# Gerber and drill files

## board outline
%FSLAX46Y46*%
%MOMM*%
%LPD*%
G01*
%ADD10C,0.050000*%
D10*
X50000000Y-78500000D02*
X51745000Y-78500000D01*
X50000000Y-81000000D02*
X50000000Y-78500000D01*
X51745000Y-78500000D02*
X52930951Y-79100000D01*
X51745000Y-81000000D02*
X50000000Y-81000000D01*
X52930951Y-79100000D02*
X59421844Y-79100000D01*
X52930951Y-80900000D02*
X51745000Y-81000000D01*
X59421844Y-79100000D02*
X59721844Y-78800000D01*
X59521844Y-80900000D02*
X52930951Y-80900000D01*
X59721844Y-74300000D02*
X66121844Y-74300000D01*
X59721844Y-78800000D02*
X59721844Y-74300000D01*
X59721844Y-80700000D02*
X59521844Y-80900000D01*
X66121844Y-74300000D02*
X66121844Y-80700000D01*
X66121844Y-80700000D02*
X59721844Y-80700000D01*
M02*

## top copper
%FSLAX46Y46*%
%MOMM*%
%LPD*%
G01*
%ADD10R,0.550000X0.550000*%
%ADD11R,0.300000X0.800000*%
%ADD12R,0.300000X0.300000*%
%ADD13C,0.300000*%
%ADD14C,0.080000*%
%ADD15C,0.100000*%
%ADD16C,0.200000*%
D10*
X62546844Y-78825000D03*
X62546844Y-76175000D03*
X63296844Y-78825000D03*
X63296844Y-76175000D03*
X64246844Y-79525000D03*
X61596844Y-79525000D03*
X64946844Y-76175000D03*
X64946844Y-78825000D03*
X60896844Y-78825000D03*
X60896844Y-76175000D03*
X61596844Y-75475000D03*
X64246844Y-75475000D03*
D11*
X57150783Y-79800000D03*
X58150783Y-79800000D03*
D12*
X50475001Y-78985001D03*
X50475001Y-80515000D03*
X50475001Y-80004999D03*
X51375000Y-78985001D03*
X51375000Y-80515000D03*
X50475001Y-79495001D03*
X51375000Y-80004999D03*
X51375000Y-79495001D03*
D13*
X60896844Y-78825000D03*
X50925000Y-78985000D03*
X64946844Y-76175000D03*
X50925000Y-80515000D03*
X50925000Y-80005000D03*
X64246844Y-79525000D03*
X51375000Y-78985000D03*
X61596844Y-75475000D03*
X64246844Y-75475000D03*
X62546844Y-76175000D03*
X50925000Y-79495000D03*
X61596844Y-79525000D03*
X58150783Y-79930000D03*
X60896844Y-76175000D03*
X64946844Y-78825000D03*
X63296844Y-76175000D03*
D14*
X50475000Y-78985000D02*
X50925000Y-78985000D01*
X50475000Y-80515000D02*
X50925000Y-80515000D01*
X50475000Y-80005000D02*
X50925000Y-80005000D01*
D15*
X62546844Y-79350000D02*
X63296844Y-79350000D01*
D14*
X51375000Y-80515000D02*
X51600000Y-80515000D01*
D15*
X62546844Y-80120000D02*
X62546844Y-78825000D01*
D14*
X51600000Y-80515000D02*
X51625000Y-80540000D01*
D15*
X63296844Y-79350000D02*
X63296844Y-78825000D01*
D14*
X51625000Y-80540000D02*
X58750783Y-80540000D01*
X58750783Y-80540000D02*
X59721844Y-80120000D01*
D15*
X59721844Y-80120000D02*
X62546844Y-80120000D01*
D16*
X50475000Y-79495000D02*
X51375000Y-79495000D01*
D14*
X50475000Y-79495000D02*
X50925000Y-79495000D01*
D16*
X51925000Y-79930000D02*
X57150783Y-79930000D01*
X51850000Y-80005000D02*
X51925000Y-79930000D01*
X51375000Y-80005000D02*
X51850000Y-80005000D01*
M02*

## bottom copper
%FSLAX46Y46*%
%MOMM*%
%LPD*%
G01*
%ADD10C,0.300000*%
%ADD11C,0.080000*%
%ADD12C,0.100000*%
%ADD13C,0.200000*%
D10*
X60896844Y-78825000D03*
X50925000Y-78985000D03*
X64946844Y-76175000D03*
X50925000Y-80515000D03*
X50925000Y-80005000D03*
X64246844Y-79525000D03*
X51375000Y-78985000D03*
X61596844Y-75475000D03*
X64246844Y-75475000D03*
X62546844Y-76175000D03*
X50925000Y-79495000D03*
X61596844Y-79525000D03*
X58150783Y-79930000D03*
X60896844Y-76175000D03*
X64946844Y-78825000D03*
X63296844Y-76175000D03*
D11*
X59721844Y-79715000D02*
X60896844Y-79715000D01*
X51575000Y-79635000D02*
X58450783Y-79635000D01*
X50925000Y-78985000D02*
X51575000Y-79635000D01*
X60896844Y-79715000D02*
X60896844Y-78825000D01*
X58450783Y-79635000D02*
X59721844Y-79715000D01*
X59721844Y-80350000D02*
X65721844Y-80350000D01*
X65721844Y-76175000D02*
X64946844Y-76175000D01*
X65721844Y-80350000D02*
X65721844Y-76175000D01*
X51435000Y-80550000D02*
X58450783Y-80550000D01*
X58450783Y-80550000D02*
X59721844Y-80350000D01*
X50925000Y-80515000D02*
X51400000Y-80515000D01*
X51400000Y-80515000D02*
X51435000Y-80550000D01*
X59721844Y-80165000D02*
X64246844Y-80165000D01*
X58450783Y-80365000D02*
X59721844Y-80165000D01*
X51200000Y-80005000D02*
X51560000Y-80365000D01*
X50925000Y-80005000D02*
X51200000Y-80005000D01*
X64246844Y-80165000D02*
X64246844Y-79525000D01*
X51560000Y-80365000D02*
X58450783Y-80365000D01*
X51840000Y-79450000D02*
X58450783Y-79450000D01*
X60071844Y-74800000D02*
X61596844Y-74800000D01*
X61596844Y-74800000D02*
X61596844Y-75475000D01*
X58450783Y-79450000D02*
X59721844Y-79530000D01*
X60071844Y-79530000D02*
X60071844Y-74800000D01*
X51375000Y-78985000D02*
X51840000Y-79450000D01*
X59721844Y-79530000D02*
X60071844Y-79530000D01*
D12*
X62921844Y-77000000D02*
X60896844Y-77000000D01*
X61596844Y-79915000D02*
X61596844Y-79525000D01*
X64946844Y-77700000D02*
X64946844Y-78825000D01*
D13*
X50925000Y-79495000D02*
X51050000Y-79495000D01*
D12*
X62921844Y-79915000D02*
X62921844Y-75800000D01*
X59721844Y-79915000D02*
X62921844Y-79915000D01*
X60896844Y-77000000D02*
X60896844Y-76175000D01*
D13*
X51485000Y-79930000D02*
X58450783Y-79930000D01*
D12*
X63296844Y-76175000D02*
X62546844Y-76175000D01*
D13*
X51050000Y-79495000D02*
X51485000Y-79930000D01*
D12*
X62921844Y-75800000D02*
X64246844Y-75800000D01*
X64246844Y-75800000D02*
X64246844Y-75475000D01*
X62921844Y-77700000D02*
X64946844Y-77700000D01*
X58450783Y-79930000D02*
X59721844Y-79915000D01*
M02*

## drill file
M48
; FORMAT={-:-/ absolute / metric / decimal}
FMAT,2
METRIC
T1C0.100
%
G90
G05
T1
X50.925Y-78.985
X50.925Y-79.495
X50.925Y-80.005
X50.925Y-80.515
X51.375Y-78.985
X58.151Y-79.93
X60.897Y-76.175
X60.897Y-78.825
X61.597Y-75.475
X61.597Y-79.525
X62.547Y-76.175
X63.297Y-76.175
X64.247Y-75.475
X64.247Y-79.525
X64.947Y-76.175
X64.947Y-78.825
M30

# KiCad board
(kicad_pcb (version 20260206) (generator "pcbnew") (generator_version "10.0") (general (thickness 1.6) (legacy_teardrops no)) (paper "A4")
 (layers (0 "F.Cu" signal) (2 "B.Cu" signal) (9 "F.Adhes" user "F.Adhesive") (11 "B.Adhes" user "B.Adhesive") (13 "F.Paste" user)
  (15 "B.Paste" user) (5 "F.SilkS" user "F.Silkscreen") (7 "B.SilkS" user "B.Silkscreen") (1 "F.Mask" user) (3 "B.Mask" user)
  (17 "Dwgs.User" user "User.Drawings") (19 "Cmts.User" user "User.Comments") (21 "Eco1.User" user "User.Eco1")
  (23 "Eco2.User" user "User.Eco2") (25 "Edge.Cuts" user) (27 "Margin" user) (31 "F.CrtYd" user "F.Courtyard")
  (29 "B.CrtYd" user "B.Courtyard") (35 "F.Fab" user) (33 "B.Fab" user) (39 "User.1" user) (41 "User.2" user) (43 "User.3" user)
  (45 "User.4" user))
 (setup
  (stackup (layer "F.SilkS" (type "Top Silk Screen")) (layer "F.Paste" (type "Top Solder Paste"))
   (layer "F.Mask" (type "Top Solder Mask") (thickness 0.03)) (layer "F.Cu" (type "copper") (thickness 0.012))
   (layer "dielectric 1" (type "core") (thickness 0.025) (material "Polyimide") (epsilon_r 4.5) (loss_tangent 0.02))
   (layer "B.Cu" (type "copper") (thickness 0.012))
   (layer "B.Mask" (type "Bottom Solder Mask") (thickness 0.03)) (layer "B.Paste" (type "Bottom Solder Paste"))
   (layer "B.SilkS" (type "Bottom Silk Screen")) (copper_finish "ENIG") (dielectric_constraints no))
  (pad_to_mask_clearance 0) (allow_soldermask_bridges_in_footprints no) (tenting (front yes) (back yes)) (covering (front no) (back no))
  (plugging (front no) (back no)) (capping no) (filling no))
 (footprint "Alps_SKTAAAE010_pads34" (layer "F.Cu") (at 62.921844 75.1)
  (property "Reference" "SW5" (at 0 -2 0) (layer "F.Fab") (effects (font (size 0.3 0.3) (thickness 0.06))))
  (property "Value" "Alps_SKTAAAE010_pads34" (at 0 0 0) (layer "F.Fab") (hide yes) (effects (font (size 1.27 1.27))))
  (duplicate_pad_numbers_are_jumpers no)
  (pad "3" smd rect (at -1.325 0.375) (size 0.55 0.55) (layers "F.Cu" "F.Mask" "F.Paste") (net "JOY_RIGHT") (solder_mask_margin 0.05)
   (thermal_bridge_angle 45))
  (pad "4" smd rect (at 1.325 0.375) (size 0.55 0.55) (layers "F.Cu" "F.Mask" "F.Paste") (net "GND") (solder_mask_margin 0.05)
   (thermal_bridge_angle 45)))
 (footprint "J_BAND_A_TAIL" (layer "F.Cu") (at 50.9 79.75)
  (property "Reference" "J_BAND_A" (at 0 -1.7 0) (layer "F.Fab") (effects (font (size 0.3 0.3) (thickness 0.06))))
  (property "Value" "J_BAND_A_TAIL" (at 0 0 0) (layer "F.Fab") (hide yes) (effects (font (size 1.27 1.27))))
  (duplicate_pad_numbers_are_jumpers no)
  (pad "1" smd rect (at -0.424999 -0.764999) (size 0.3 0.3) (layers "F.Cu" "F.Mask") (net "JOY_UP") (solder_mask_margin 0.05)
   (thermal_bridge_angle 45))
  (pad "2" smd rect (at -0.424999 0.765) (size 0.3 0.3) (layers "F.Cu" "F.Mask") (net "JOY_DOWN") (solder_mask_margin 0.05)
   (thermal_bridge_angle 45))
  (pad "3" smd rect (at -0.424999 0.254999) (size 0.3 0.3) (layers "F.Cu" "F.Mask") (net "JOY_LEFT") (solder_mask_margin 0.05)
   (thermal_bridge_angle 45))
  (pad "4" smd rect (at 0.475 -0.764999) (size 0.3 0.3) (layers "F.Cu" "F.Mask") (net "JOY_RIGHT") (solder_mask_margin 0.05)
   (thermal_bridge_angle 45))
  (pad "5" smd rect (at 0.475 0.765) (size 0.3 0.3) (layers "F.Cu" "F.Mask") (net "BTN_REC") (solder_mask_margin 0.05)
   (thermal_bridge_angle 45))
  (pad "6" smd rect (at -0.424999 -0.254999) (size 0.3 0.3) (layers "F.Cu" "F.Mask") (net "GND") (solder_mask_margin 0.05)
   (thermal_bridge_angle 45))
  (pad "7" smd rect (at 0.475 0.254999) (size 0.3 0.3) (layers "F.Cu" "F.Mask") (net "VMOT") (solder_mask_margin 0.05)
   (thermal_bridge_angle 45))
  (pad "8" smd rect (at 0.475 -0.254999) (size 0.3 0.3) (layers "F.Cu" "F.Mask") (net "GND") (solder_mask_margin 0.05)
   (thermal_bridge_angle 45)))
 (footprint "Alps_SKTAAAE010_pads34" (layer "F.Cu") (at 62.921844 79.9 180)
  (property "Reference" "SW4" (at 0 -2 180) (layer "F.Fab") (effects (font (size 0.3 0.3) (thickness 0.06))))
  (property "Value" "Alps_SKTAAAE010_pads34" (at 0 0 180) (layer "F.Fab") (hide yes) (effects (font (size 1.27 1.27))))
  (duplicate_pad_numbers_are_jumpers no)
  (pad "3" smd rect (at -1.325 0.375 180) (size 0.55 0.55) (layers "F.Cu" "F.Mask" "F.Paste") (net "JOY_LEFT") (solder_mask_margin 0.05)
   (thermal_bridge_angle 45))
  (pad "4" smd rect (at 1.325 0.375 180) (size 0.55 0.55) (layers "F.Cu" "F.Mask" "F.Paste") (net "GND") (solder_mask_margin 0.05)
   (thermal_bridge_angle 45)))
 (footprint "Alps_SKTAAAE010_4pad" (layer "F.Cu") (at 62.921844 77.5 90)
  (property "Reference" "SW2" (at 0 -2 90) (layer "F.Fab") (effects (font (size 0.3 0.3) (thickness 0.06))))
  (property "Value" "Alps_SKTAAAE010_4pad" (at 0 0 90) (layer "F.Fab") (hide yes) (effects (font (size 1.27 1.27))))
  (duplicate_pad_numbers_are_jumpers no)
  (pad "1" smd rect (at -1.325 -0.375 90) (size 0.55 0.55) (layers "F.Cu" "F.Mask" "F.Paste") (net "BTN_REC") (solder_mask_margin 0.05)
   (thermal_bridge_angle 45))
  (pad "2" smd rect (at 1.325 -0.375 90) (size 0.55 0.55) (layers "F.Cu" "F.Mask" "F.Paste") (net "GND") (solder_mask_margin 0.05)
   (thermal_bridge_angle 45))
  (pad "3" smd rect (at -1.325 0.375 90) (size 0.55 0.55) (layers "F.Cu" "F.Mask" "F.Paste") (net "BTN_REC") (solder_mask_margin 0.05)
   (thermal_bridge_angle 45))
  (pad "4" smd rect (at 1.325 0.375 90) (size 0.55 0.55) (layers "F.Cu" "F.Mask" "F.Paste") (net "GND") (solder_mask_margin 0.05)
   (thermal_bridge_angle 45)))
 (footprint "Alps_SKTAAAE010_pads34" (layer "F.Cu") (at 65.321844 77.5 -90)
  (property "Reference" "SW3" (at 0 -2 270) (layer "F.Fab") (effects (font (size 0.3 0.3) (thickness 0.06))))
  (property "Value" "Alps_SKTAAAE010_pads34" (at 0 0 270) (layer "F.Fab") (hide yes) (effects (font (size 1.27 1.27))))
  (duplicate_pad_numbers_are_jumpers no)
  (pad "3" smd rect (at -1.325 0.375 270) (size 0.55 0.55) (layers "F.Cu" "F.Mask" "F.Paste") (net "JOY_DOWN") (solder_mask_margin 0.05)
   (thermal_bridge_angle 45))
  (pad "4" smd rect (at 1.325 0.375 270) (size 0.55 0.55) (layers "F.Cu" "F.Mask" "F.Paste") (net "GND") (solder_mask_margin 0.05)
   (thermal_bridge_angle 45)))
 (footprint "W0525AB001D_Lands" (layer "F.Cu") (at 57.650783 79.93)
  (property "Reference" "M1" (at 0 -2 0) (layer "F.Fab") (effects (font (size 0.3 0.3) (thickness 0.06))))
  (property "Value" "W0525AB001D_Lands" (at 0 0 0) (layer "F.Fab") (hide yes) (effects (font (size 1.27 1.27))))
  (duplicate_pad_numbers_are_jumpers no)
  (pad "1" smd rect (at -0.5 -0.13) (size 0.3 0.8) (layers "F.Cu" "F.Mask") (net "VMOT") (solder_mask_margin 0.05) (thermal_bridge_angle 45))
  (pad "2" smd rect (at 0.5 -0.13) (size 0.3 0.8) (layers "F.Cu" "F.Mask") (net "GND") (solder_mask_margin 0.05) (thermal_bridge_angle 45)))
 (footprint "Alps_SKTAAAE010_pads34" (layer "F.Cu") (at 60.521844 77.5 90)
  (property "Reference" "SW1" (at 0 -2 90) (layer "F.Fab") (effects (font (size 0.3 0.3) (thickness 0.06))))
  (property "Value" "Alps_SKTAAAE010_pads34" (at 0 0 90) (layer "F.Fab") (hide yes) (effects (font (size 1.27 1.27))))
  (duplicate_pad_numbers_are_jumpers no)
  (pad "3" smd rect (at -1.325 0.375 90) (size 0.55 0.55) (layers "F.Cu" "F.Mask" "F.Paste") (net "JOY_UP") (solder_mask_margin 0.05)
   (thermal_bridge_angle 45))
  (pad "4" smd rect (at 1.325 0.375 90) (size 0.55 0.55) (layers "F.Cu" "F.Mask" "F.Paste") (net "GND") (solder_mask_margin 0.05)
   (thermal_bridge_angle 45)))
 (gr_line (start 50 78.5) (end 51.745 78.5) (stroke (width 0.05) (type default)) (layer "Edge.Cuts"))
 (gr_line (start 50 81) (end 50 78.5) (stroke (width 0.05) (type default)) (layer "Edge.Cuts"))
 (gr_line (start 51.745 78.5) (end 52.930951 79.1) (stroke (width 0.05) (type default)) (layer "Edge.Cuts"))
 (gr_line (start 51.745 81) (end 50 81) (stroke (width 0.05) (type default)) (layer "Edge.Cuts"))
 (gr_line (start 52.930951 79.1) (end 59.421844 79.1) (stroke (width 0.05) (type default)) (layer "Edge.Cuts"))
 (gr_line (start 52.930951 80.9) (end 51.745 81) (stroke (width 0.05) (type default)) (layer "Edge.Cuts"))
 (gr_line (start 59.421844 79.1) (end 59.721844 78.8) (stroke (width 0.05) (type default)) (layer "Edge.Cuts"))
 (gr_line (start 59.521844 80.9) (end 52.930951 80.9) (stroke (width 0.05) (type default)) (layer "Edge.Cuts"))
 (gr_line (start 59.721844 74.3) (end 66.121844 74.3) (stroke (width 0.05) (type default)) (layer "Edge.Cuts"))
 (gr_line (start 59.721844 78.8) (end 59.721844 74.3) (stroke (width 0.05) (type default)) (layer "Edge.Cuts"))
 (gr_line (start 59.721844 80.7) (end 59.521844 80.9) (stroke (width 0.05) (type default)) (layer "Edge.Cuts"))
 (gr_line (start 66.121844 74.3) (end 66.121844 80.7) (stroke (width 0.05) (type default)) (layer "Edge.Cuts"))
 (gr_line (start 66.121844 80.7) (end 59.721844 80.7) (stroke (width 0.05) (type default)) (layer "Edge.Cuts"))
 (via (at 51.375 78.985) (size 0.3) (drill 0.1) (layers "F.Cu" "B.Cu") (tenting (front yes) (back yes)) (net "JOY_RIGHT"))
 (via (at 61.596844 75.475) (size 0.3) (drill 0.1) (layers "F.Cu" "B.Cu") (tenting (front yes) (back yes)) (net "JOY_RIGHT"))
 (segment (start 59.721844 79.53) (end 60.071844 79.53) (width 0.08) (layer "B.Cu") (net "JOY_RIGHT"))
 (segment (start 51.375 78.985) (end 51.84 79.45) (width 0.08) (layer "B.Cu") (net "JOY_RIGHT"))
 (segment (start 51.84 79.45) (end 58.450783 79.45) (width 0.08) (layer "B.Cu") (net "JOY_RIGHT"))
 (segment (start 58.450783 79.45) (end 59.721844 79.53) (width 0.08) (layer "B.Cu") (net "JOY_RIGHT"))
 (segment (start 61.596844 74.8) (end 61.596844 75.475) (width 0.08) (layer "B.Cu") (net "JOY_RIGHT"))
 (segment (start 60.071844 79.53) (end 60.071844 74.8) (width 0.08) (layer "B.Cu") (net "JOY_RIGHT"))
 (segment (start 60.071844 74.8) (end 61.596844 74.8) (width 0.08) (layer "B.Cu") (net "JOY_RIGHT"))
 (segment (start 50.475 79.495) (end 50.925 79.495) (width 0.08) (layer "F.Cu") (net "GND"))
 (segment (start 50.475 79.495) (end 51.375 79.495) (width 0.2) (layer "F.Cu") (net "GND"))
 (via (at 60.896844 76.175) (size 0.3) (drill 0.1) (layers "F.Cu" "B.Cu") (tenting (front yes) (back yes)) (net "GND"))
 (via (at 63.296844 76.175) (size 0.3) (drill 0.1) (layers "F.Cu" "B.Cu") (tenting (front yes) (back yes)) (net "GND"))
 (via (at 64.246844 75.475) (size 0.3) (drill 0.1) (layers "F.Cu" "B.Cu") (tenting (front yes) (back yes)) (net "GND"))
 (via (at 64.946844 78.825) (size 0.3) (drill 0.1) (layers "F.Cu" "B.Cu") (tenting (front yes) (back yes)) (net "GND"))
 (via (at 62.546844 76.175) (size 0.3) (drill 0.1) (layers "F.Cu" "B.Cu") (tenting (front yes) (back yes)) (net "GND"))
 (via (at 58.150783 79.93) (size 0.3) (drill 0.1) (layers "F.Cu" "B.Cu") (tenting (front yes) (back yes)) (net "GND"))
 (via (at 61.596844 79.525) (size 0.3) (drill 0.1) (layers "F.Cu" "B.Cu") (tenting (front yes) (back yes)) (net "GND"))
 (via (at 50.925 79.495) (size 0.3) (drill 0.1) (layers "F.Cu" "B.Cu") (tenting (front yes) (back yes)) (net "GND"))
 (segment (start 64.946844 77.7) (end 64.946844 78.825) (width 0.1) (layer "B.Cu") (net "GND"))
 (segment (start 63.296844 76.175) (end 62.546844 76.175) (width 0.1) (layer "B.Cu") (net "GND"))
 (segment (start 60.896844 77) (end 60.896844 76.175) (width 0.1) (layer "B.Cu") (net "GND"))
 (segment (start 50.925 79.495) (end 51.05 79.495) (width 0.2) (layer "B.Cu") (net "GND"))
 (segment (start 62.921844 77) (end 60.896844 77) (width 0.1) (layer "B.Cu") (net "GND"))
 (segment (start 61.596844 79.915) (end 61.596844 79.525) (width 0.1) (layer "B.Cu") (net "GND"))
 (segment (start 58.450783 79.93) (end 59.721844 79.915) (width 0.1) (layer "B.Cu") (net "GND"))
 (segment (start 51.05 79.495) (end 51.485 79.93) (width 0.2) (layer "B.Cu") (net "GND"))
 (segment (start 62.921844 75.8) (end 64.246844 75.8) (width 0.1) (layer "B.Cu") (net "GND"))
 (segment (start 64.246844 75.8) (end 64.246844 75.475) (width 0.1) (layer "B.Cu") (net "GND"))
 (segment (start 51.485 79.93) (end 58.450783 79.93) (width 0.2) (layer "B.Cu") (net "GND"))
 (segment (start 62.921844 77.7) (end 64.946844 77.7) (width 0.1) (layer "B.Cu") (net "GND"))
 (segment (start 59.721844 79.915) (end 62.921844 79.915) (width 0.1) (layer "B.Cu") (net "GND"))
 (segment (start 62.921844 79.915) (end 62.921844 75.8) (width 0.1) (layer "B.Cu") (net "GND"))
 (segment (start 50.475 78.985) (end 50.925 78.985) (width 0.08) (layer "F.Cu") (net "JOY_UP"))
 (via (at 60.896844 78.825) (size 0.3) (drill 0.1) (layers "F.Cu" "B.Cu") (tenting (front yes) (back yes)) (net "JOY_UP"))
 (via (at 50.925 78.985) (size 0.3) (drill 0.1) (layers "F.Cu" "B.Cu") (tenting (front yes) (back yes)) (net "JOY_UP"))
 (segment (start 58.450783 79.635) (end 59.721844 79.715) (width 0.08) (layer "B.Cu") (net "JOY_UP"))
 (segment (start 51.575 79.635) (end 58.450783 79.635) (width 0.08) (layer "B.Cu") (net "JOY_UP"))
 (segment (start 50.925 78.985) (end 51.575 79.635) (width 0.08) (layer "B.Cu") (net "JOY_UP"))
 (segment (start 60.896844 79.715) (end 60.896844 78.825) (width 0.08) (layer "B.Cu") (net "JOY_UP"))
 (segment (start 59.721844 79.715) (end 60.896844 79.715) (width 0.08) (layer "B.Cu") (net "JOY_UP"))
 (segment (start 50.475 80.515) (end 50.925 80.515) (width 0.08) (layer "F.Cu") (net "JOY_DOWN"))
 (via (at 50.925 80.515) (size 0.3) (drill 0.1) (layers "F.Cu" "B.Cu") (tenting (front yes) (back yes)) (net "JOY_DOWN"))
 (via (at 64.946844 76.175) (size 0.3) (drill 0.1) (layers "F.Cu" "B.Cu") (tenting (front yes) (back yes)) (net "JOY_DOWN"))
 (segment (start 59.721844 80.35) (end 65.721844 80.35) (width 0.08) (layer "B.Cu") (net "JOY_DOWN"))
 (segment (start 65.721844 76.175) (end 64.946844 76.175) (width 0.08) (layer "B.Cu") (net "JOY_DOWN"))
 (segment (start 50.925 80.515) (end 51.4 80.515) (width 0.08) (layer "B.Cu") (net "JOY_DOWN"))
 (segment (start 58.450783 80.55) (end 59.721844 80.35) (width 0.08) (layer "B.Cu") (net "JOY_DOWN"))
 (segment (start 65.721844 80.35) (end 65.721844 76.175) (width 0.08) (layer "B.Cu") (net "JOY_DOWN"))
 (segment (start 51.4 80.515) (end 51.435 80.55) (width 0.08) (layer "B.Cu") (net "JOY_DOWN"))
 (segment (start 51.435 80.55) (end 58.450783 80.55) (width 0.08) (layer "B.Cu") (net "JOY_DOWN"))
 (segment (start 50.475 80.005) (end 50.925 80.005) (width 0.08) (layer "F.Cu") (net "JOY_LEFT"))
 (via (at 64.246844 79.525) (size 0.3) (drill 0.1) (layers "F.Cu" "B.Cu") (tenting (front yes) (back yes)) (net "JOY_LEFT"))
 (via (at 50.925 80.005) (size 0.3) (drill 0.1) (layers "F.Cu" "B.Cu") (tenting (front yes) (back yes)) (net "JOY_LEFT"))
 (segment (start 51.2 80.005) (end 51.56 80.365) (width 0.08) (layer "B.Cu") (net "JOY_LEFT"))
 (segment (start 59.721844 80.165) (end 64.246844 80.165) (width 0.08) (layer "B.Cu") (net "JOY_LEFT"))
 (segment (start 64.246844 80.165) (end 64.246844 79.525) (width 0.08) (layer "B.Cu") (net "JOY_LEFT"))
 (segment (start 58.450783 80.365) (end 59.721844 80.165) (width 0.08) (layer "B.Cu") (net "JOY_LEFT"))
 (segment (start 50.925 80.005) (end 51.2 80.005) (width 0.08) (layer "B.Cu") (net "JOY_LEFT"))
 (segment (start 51.56 80.365) (end 58.450783 80.365) (width 0.08) (layer "B.Cu") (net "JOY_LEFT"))
 (segment (start 62.546844 79.35) (end 63.296844 79.35) (width 0.1) (layer "F.Cu") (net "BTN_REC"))
 (segment (start 63.296844 79.35) (end 63.296844 78.825) (width 0.1) (layer "F.Cu") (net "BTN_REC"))
 (segment (start 51.375 80.515) (end 51.6 80.515) (width 0.08) (layer "F.Cu") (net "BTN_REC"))
 (segment (start 58.750783 80.54) (end 59.721844 80.12) (width 0.08) (layer "F.Cu") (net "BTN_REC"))
 (segment (start 51.6 80.515) (end 51.625 80.54) (width 0.08) (layer "F.Cu") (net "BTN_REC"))
 (segment (start 59.721844 80.12) (end 62.546844 80.12) (width 0.1) (layer "F.Cu") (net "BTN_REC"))
 (segment (start 51.625 80.54) (end 58.750783 80.54) (width 0.08) (layer "F.Cu") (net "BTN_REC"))
 (segment (start 62.546844 80.12) (end 62.546844 78.825) (width 0.1) (layer "F.Cu") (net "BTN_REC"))
 (segment (start 51.925 79.93) (end 57.150783 79.93) (width 0.2) (layer "F.Cu") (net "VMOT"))
 (segment (start 51.375 80.005) (end 51.85 80.005) (width 0.2) (layer "F.Cu") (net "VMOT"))
 (segment (start 51.85 80.005) (end 51.925 79.93) (width 0.2) (layer "F.Cu") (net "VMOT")))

